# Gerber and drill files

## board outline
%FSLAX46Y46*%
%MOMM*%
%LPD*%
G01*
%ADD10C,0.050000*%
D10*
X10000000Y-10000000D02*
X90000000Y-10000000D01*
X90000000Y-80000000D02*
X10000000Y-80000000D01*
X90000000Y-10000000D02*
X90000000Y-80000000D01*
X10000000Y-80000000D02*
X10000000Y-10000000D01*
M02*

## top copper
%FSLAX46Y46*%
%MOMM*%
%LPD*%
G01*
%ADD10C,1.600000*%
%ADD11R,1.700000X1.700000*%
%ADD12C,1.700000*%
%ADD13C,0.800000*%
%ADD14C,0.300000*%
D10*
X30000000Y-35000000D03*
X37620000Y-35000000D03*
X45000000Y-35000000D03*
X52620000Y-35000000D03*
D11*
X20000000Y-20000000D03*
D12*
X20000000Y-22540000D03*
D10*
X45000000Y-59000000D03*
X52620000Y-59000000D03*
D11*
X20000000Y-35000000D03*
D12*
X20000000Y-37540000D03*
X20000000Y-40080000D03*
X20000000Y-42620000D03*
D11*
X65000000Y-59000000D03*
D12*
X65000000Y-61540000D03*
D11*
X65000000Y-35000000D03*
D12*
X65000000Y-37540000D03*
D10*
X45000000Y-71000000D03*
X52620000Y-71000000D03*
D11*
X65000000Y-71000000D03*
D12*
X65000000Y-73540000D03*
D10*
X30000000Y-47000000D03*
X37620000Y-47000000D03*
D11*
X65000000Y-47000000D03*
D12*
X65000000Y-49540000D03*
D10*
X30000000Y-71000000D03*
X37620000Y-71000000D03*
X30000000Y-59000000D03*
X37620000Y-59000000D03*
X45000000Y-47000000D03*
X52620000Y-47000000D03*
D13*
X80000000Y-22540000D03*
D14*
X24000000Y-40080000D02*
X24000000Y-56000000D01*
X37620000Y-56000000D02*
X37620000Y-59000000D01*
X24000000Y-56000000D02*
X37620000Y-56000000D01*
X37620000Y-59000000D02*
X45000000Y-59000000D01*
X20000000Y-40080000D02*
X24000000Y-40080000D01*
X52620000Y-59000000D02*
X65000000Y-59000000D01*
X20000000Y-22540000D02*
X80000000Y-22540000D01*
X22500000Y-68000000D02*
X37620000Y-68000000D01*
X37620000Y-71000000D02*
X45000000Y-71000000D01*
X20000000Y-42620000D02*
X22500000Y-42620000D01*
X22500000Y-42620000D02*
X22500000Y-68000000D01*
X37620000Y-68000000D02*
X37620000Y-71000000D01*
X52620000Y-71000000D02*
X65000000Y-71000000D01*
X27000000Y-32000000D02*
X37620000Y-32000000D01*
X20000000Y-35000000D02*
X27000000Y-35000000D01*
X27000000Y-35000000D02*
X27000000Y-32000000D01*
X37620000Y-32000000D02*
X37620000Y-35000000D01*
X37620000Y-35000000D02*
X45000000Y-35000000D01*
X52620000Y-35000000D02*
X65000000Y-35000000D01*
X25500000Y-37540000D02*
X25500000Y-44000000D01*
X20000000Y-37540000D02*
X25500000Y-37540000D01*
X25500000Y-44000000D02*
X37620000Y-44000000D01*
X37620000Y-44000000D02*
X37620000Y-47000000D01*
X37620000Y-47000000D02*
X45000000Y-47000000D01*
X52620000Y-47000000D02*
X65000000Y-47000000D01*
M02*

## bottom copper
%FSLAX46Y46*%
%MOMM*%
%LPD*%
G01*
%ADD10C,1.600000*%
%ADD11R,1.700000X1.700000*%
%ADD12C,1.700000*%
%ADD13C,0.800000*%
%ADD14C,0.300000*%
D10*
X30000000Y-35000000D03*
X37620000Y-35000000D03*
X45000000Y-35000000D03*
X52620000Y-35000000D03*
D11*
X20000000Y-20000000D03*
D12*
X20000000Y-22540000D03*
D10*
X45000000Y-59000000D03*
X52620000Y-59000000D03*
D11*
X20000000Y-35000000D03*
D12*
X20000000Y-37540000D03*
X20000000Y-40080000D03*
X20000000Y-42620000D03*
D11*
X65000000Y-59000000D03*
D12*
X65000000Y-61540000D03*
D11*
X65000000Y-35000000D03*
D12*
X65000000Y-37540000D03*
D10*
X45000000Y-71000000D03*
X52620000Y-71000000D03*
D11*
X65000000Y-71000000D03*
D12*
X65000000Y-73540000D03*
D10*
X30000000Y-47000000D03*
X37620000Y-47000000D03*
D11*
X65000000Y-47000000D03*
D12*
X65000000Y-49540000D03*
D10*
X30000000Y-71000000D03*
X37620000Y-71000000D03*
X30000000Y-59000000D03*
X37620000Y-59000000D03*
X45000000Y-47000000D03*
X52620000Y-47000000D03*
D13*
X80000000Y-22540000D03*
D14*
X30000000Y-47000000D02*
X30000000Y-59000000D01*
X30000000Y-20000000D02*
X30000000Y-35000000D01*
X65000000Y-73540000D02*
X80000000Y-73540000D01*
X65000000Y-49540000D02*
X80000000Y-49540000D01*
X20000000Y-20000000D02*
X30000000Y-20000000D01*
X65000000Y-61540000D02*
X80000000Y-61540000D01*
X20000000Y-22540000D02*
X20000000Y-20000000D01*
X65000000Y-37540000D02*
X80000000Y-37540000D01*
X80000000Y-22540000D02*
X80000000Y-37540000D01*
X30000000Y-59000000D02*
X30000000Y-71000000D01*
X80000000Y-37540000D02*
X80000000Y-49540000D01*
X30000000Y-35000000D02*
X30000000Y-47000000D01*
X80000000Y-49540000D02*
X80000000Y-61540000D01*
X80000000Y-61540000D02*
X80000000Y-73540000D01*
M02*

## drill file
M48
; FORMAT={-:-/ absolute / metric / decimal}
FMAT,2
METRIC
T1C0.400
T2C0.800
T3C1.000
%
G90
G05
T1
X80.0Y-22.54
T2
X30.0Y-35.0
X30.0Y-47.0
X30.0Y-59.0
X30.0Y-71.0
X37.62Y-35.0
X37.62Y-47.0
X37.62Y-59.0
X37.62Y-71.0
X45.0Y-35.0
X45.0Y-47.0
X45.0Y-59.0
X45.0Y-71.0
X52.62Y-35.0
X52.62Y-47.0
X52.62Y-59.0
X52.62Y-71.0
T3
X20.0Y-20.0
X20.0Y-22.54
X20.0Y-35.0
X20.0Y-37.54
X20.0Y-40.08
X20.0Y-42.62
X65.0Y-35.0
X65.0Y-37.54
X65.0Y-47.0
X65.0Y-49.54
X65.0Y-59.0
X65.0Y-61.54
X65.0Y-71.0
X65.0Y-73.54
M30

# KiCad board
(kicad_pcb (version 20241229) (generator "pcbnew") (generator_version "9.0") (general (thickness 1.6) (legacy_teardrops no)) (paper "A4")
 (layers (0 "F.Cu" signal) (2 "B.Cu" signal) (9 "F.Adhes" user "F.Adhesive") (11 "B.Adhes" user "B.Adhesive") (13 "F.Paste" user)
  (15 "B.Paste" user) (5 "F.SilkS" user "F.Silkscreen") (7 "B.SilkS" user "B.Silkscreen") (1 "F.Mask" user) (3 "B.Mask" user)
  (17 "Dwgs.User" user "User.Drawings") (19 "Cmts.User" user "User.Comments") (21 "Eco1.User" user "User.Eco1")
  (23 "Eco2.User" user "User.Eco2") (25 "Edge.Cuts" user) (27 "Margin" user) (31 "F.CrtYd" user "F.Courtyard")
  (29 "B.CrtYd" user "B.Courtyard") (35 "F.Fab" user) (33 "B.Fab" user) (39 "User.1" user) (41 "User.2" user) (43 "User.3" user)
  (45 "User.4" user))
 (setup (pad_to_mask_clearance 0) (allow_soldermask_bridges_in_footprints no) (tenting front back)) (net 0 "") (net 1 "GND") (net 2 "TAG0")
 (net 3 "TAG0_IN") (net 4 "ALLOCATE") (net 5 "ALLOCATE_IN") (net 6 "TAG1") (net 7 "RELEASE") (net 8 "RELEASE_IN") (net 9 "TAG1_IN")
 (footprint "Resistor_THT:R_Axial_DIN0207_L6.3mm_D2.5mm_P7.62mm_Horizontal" (layer "F.Cu") (at 30 35)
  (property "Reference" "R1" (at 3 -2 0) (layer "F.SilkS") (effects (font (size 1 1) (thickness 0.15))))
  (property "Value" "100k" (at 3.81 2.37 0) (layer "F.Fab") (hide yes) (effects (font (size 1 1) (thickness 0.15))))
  (pad "1" thru_hole circle (at 0 0) (size 1.6 1.6) (drill 0.8) (layers "*.Cu" "*.Mask") (remove_unused_layers no) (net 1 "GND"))
  (pad "2" thru_hole circle (at 7.62 0) (size 1.6 1.6) (drill 0.8) (layers "*.Cu" "*.Mask") (remove_unused_layers no) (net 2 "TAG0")))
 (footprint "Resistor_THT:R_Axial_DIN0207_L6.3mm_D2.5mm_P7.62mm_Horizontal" (layer "F.Cu") (at 45 35)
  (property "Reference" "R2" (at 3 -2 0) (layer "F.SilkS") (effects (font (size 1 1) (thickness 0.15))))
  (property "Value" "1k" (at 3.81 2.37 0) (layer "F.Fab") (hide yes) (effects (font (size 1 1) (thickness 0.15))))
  (pad "1" thru_hole circle (at 0 0) (size 1.6 1.6) (drill 0.8) (layers "*.Cu" "*.Mask") (remove_unused_layers no) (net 2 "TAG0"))
  (pad "2" thru_hole circle (at 7.62 0) (size 1.6 1.6) (drill 0.8) (layers "*.Cu" "*.Mask") (remove_unused_layers no) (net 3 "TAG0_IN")))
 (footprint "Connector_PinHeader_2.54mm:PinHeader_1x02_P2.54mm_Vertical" (layer "F.Cu") (at 20 20)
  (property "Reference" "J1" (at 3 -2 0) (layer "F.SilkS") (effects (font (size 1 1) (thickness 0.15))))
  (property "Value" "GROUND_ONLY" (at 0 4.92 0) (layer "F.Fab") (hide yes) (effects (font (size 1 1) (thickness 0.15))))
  (pad "1" thru_hole rect (at 0 0) (size 1.7 1.7) (drill 1) (layers "*.Cu" "*.Mask") (remove_unused_layers no) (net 1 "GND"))
  (pad "2" thru_hole circle (at 0 2.54) (size 1.7 1.7) (drill 1) (layers "*.Cu" "*.Mask") (remove_unused_layers no) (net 1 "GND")))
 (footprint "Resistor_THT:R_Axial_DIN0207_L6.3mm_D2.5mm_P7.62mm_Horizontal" (layer "F.Cu") (at 45 59)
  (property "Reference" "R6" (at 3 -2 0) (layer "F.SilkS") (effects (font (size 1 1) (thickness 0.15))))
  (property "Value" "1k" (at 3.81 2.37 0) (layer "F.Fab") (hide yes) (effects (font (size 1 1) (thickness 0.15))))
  (pad "1" thru_hole circle (at 0 0) (size 1.6 1.6) (drill 0.8) (layers "*.Cu" "*.Mask") (remove_unused_layers no) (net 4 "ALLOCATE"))
  (pad "2" thru_hole circle (at 7.62 0) (size 1.6 1.6) (drill 0.8) (layers "*.Cu" "*.Mask") (remove_unused_layers no) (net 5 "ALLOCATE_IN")))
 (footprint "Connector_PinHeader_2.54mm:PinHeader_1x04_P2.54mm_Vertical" (layer "F.Cu") (at 20 35)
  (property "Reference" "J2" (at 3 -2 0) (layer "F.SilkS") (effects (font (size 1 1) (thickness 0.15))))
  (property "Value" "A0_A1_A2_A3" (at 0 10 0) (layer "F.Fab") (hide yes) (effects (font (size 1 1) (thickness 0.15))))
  (pad "1" thru_hole rect (at 0 0) (size 1.7 1.7) (drill 1) (layers "*.Cu" "*.Mask") (remove_unused_layers no) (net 2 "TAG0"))
  (pad "2" thru_hole circle (at 0 2.54) (size 1.7 1.7) (drill 1) (layers "*.Cu" "*.Mask") (remove_unused_layers no) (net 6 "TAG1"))
  (pad "3" thru_hole circle (at 0 5.08) (size 1.7 1.7) (drill 1) (layers "*.Cu" "*.Mask") (remove_unused_layers no) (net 4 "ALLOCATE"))
  (pad "4" thru_hole circle (at 0 7.62) (size 1.7 1.7) (drill 1) (layers "*.Cu" "*.Mask") (remove_unused_layers no) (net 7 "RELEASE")))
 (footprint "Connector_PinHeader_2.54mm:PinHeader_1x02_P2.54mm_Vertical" (layer "F.Cu") (at 65 59)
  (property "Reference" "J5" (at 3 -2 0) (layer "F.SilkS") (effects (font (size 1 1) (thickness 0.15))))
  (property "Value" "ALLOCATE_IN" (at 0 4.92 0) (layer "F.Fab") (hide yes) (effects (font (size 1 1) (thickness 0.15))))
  (pad "1" thru_hole rect (at 0 0) (size 1.7 1.7) (drill 1) (layers "*.Cu" "*.Mask") (remove_unused_layers no) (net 5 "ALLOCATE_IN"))
  (pad "2" thru_hole circle (at 0 2.54) (size 1.7 1.7) (drill 1) (layers "*.Cu" "*.Mask") (remove_unused_layers no) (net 1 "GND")))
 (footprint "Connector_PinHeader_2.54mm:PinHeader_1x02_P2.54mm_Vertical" (layer "F.Cu") (at 65 35)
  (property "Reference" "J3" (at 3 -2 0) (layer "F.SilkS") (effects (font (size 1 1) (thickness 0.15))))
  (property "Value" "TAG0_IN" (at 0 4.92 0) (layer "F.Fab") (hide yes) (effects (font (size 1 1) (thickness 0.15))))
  (pad "1" thru_hole rect (at 0 0) (size 1.7 1.7) (drill 1) (layers "*.Cu" "*.Mask") (remove_unused_layers no) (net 3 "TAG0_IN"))
  (pad "2" thru_hole circle (at 0 2.54) (size 1.7 1.7) (drill 1) (layers "*.Cu" "*.Mask") (remove_unused_layers no) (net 1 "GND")))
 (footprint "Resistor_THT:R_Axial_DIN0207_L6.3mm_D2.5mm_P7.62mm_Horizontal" (layer "F.Cu") (at 45 71)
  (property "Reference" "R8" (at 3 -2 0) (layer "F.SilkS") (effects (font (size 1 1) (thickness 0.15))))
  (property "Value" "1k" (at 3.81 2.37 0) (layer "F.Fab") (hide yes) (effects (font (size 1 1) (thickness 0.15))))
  (pad "1" thru_hole circle (at 0 0) (size 1.6 1.6) (drill 0.8) (layers "*.Cu" "*.Mask") (remove_unused_layers no) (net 7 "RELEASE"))
  (pad "2" thru_hole circle (at 7.62 0) (size 1.6 1.6) (drill 0.8) (layers "*.Cu" "*.Mask") (remove_unused_layers no) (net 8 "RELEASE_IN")))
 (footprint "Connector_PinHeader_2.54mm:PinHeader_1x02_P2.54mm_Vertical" (layer "F.Cu") (at 65 71)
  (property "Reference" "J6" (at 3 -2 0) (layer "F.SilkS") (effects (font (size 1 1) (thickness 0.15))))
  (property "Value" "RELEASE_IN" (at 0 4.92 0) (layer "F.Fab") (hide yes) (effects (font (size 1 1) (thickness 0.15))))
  (pad "1" thru_hole rect (at 0 0) (size 1.7 1.7) (drill 1) (layers "*.Cu" "*.Mask") (remove_unused_layers no) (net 8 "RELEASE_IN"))
  (pad "2" thru_hole circle (at 0 2.54) (size 1.7 1.7) (drill 1) (layers "*.Cu" "*.Mask") (remove_unused_layers no) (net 1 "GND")))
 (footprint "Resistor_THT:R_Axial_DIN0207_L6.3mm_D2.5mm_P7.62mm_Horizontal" (layer "F.Cu") (at 30 47)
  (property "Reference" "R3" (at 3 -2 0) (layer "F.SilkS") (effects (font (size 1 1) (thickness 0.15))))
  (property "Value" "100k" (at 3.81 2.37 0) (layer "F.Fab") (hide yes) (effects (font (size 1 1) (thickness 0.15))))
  (pad "1" thru_hole circle (at 0 0) (size 1.6 1.6) (drill 0.8) (layers "*.Cu" "*.Mask") (remove_unused_layers no) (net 1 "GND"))
  (pad "2" thru_hole circle (at 7.62 0) (size 1.6 1.6) (drill 0.8) (layers "*.Cu" "*.Mask") (remove_unused_layers no) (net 6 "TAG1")))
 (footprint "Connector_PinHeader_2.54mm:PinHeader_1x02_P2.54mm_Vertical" (layer "F.Cu") (at 65 47)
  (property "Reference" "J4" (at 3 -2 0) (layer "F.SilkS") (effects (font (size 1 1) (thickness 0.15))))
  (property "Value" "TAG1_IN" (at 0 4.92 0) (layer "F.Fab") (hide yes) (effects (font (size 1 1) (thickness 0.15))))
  (pad "1" thru_hole rect (at 0 0) (size 1.7 1.7) (drill 1) (layers "*.Cu" "*.Mask") (remove_unused_layers no) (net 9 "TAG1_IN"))
  (pad "2" thru_hole circle (at 0 2.54) (size 1.7 1.7) (drill 1) (layers "*.Cu" "*.Mask") (remove_unused_layers no) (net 1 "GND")))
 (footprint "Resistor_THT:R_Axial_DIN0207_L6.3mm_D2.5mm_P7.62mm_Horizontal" (layer "F.Cu") (at 30 71)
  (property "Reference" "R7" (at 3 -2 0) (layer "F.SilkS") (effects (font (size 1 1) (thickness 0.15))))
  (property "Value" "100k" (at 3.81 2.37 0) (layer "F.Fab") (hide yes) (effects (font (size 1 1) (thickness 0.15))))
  (pad "1" thru_hole circle (at 0 0) (size 1.6 1.6) (drill 0.8) (layers "*.Cu" "*.Mask") (remove_unused_layers no) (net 1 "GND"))
  (pad "2" thru_hole circle (at 7.62 0) (size 1.6 1.6) (drill 0.8) (layers "*.Cu" "*.Mask") (remove_unused_layers no) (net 7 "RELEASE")))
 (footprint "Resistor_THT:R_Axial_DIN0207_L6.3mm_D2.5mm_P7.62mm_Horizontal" (layer "F.Cu") (at 30 59)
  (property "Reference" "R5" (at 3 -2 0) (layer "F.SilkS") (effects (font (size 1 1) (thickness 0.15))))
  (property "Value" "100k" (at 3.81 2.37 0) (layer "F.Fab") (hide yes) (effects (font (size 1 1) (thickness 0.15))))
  (pad "1" thru_hole circle (at 0 0) (size 1.6 1.6) (drill 0.8) (layers "*.Cu" "*.Mask") (remove_unused_layers no) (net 1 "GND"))
  (pad "2" thru_hole circle (at 7.62 0) (size 1.6 1.6) (drill 0.8) (layers "*.Cu" "*.Mask") (remove_unused_layers no) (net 4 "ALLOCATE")))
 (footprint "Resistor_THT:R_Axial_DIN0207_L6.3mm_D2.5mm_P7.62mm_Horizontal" (layer "F.Cu") (at 45 47)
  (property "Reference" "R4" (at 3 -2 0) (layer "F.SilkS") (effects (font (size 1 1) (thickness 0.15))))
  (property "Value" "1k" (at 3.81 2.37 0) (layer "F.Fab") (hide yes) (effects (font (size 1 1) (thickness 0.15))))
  (pad "1" thru_hole circle (at 0 0) (size 1.6 1.6) (drill 0.8) (layers "*.Cu" "*.Mask") (remove_unused_layers no) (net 6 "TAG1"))
  (pad "2" thru_hole circle (at 7.62 0) (size 1.6 1.6) (drill 0.8) (layers "*.Cu" "*.Mask") (remove_unused_layers no) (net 9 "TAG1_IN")))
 (gr_line (start 10 10) (end 90 10) (stroke (width 0.05) (type default)) (layer "Edge.Cuts"))
 (gr_line (start 90 80) (end 10 80) (stroke (width 0.05) (type default)) (layer "Edge.Cuts"))
 (gr_line (start 90 10) (end 90 80) (stroke (width 0.05) (type default)) (layer "Edge.Cuts"))
 (gr_line (start 10 80) (end 10 10) (stroke (width 0.05) (type default)) (layer "Edge.Cuts"))
 (segment (start 24 40.08) (end 24 56) (width 0.3) (layer "F.Cu") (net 4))
 (segment (start 37.62 56) (end 37.62 59) (width 0.3) (layer "F.Cu") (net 4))
 (segment (start 24 56) (end 37.62 56) (width 0.3) (layer "F.Cu") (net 4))
 (segment (start 37.62 59) (end 45 59) (width 0.3) (layer "F.Cu") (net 4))
 (segment (start 20 40.08) (end 24 40.08) (width 0.3) (layer "F.Cu") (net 4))
 (segment (start 52.62 59) (end 65 59) (width 0.3) (layer "F.Cu") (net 5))
 (segment (start 20 22.54) (end 80 22.54) (width 0.3) (layer "F.Cu") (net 1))
 (via (at 80 22.54) (size 0.8) (drill 0.4) (layers "F.Cu" "B.Cu") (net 1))
 (segment (start 30 47) (end 30 59) (width 0.3) (layer "B.Cu") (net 1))
 (segment (start 30 20) (end 30 35) (width 0.3) (layer "B.Cu") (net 1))
 (segment (start 65 73.54) (end 80 73.54) (width 0.3) (layer "B.Cu") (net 1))
 (segment (start 65 49.54) (end 80 49.54) (width 0.3) (layer "B.Cu") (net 1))
 (segment (start 20 20) (end 30 20) (width 0.3) (layer "B.Cu") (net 1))
 (segment (start 65 61.54) (end 80 61.54) (width 0.3) (layer "B.Cu") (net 1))
 (segment (start 20 22.54) (end 20 20) (width 0.3) (layer "B.Cu") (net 1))
 (segment (start 65 37.54) (end 80 37.54) (width 0.3) (layer "B.Cu") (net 1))
 (segment (start 80 22.54) (end 80 37.54) (width 0.3) (layer "B.Cu") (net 1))
 (segment (start 30 59) (end 30 71) (width 0.3) (layer "B.Cu") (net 1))
 (segment (start 80 37.54) (end 80 49.54) (width 0.3) (layer "B.Cu") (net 1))
 (segment (start 30 35) (end 30 47) (width 0.3) (layer "B.Cu") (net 1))
 (segment (start 80 49.54) (end 80 61.54) (width 0.3) (layer "B.Cu") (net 1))
 (segment (start 80 61.54) (end 80 73.54) (width 0.3) (layer "B.Cu") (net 1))
 (segment (start 22.5 68) (end 37.62 68) (width 0.3) (layer "F.Cu") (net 7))
 (segment (start 37.62 71) (end 45 71) (width 0.3) (layer "F.Cu") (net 7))
 (segment (start 20 42.62) (end 22.5 42.62) (width 0.3) (layer "F.Cu") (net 7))
 (segment (start 22.5 42.62) (end 22.5 68) (width 0.3) (layer "F.Cu") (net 7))
 (segment (start 37.62 68) (end 37.62 71) (width 0.3) (layer "F.Cu") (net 7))
 (segment (start 52.62 71) (end 65 71) (width 0.3) (layer "F.Cu") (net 8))
 (segment (start 27 32) (end 37.62 32) (width 0.3) (layer "F.Cu") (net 2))
 (segment (start 20 35) (end 27 35) (width 0.3) (layer "F.Cu") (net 2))
 (segment (start 27 35) (end 27 32) (width 0.3) (layer "F.Cu") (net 2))
 (segment (start 37.62 32) (end 37.62 35) (width 0.3) (layer "F.Cu") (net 2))
 (segment (start 37.62 35) (end 45 35) (width 0.3) (layer "F.Cu") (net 2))
 (segment (start 52.62 35) (end 65 35) (width 0.3) (layer "F.Cu") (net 3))
 (segment (start 25.5 37.54) (end 25.5 44) (width 0.3) (layer "F.Cu") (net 6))
 (segment (start 20 37.54) (end 25.5 37.54) (width 0.3) (layer "F.Cu") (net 6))
 (segment (start 25.5 44) (end 37.62 44) (width 0.3) (layer "F.Cu") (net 6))
 (segment (start 37.62 44) (end 37.62 47) (width 0.3) (layer "F.Cu") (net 6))
 (segment (start 37.62 47) (end 45 47) (width 0.3) (layer "F.Cu") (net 6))
 (segment (start 52.62 47) (end 65 47) (width 0.3) (layer "F.Cu") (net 9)))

